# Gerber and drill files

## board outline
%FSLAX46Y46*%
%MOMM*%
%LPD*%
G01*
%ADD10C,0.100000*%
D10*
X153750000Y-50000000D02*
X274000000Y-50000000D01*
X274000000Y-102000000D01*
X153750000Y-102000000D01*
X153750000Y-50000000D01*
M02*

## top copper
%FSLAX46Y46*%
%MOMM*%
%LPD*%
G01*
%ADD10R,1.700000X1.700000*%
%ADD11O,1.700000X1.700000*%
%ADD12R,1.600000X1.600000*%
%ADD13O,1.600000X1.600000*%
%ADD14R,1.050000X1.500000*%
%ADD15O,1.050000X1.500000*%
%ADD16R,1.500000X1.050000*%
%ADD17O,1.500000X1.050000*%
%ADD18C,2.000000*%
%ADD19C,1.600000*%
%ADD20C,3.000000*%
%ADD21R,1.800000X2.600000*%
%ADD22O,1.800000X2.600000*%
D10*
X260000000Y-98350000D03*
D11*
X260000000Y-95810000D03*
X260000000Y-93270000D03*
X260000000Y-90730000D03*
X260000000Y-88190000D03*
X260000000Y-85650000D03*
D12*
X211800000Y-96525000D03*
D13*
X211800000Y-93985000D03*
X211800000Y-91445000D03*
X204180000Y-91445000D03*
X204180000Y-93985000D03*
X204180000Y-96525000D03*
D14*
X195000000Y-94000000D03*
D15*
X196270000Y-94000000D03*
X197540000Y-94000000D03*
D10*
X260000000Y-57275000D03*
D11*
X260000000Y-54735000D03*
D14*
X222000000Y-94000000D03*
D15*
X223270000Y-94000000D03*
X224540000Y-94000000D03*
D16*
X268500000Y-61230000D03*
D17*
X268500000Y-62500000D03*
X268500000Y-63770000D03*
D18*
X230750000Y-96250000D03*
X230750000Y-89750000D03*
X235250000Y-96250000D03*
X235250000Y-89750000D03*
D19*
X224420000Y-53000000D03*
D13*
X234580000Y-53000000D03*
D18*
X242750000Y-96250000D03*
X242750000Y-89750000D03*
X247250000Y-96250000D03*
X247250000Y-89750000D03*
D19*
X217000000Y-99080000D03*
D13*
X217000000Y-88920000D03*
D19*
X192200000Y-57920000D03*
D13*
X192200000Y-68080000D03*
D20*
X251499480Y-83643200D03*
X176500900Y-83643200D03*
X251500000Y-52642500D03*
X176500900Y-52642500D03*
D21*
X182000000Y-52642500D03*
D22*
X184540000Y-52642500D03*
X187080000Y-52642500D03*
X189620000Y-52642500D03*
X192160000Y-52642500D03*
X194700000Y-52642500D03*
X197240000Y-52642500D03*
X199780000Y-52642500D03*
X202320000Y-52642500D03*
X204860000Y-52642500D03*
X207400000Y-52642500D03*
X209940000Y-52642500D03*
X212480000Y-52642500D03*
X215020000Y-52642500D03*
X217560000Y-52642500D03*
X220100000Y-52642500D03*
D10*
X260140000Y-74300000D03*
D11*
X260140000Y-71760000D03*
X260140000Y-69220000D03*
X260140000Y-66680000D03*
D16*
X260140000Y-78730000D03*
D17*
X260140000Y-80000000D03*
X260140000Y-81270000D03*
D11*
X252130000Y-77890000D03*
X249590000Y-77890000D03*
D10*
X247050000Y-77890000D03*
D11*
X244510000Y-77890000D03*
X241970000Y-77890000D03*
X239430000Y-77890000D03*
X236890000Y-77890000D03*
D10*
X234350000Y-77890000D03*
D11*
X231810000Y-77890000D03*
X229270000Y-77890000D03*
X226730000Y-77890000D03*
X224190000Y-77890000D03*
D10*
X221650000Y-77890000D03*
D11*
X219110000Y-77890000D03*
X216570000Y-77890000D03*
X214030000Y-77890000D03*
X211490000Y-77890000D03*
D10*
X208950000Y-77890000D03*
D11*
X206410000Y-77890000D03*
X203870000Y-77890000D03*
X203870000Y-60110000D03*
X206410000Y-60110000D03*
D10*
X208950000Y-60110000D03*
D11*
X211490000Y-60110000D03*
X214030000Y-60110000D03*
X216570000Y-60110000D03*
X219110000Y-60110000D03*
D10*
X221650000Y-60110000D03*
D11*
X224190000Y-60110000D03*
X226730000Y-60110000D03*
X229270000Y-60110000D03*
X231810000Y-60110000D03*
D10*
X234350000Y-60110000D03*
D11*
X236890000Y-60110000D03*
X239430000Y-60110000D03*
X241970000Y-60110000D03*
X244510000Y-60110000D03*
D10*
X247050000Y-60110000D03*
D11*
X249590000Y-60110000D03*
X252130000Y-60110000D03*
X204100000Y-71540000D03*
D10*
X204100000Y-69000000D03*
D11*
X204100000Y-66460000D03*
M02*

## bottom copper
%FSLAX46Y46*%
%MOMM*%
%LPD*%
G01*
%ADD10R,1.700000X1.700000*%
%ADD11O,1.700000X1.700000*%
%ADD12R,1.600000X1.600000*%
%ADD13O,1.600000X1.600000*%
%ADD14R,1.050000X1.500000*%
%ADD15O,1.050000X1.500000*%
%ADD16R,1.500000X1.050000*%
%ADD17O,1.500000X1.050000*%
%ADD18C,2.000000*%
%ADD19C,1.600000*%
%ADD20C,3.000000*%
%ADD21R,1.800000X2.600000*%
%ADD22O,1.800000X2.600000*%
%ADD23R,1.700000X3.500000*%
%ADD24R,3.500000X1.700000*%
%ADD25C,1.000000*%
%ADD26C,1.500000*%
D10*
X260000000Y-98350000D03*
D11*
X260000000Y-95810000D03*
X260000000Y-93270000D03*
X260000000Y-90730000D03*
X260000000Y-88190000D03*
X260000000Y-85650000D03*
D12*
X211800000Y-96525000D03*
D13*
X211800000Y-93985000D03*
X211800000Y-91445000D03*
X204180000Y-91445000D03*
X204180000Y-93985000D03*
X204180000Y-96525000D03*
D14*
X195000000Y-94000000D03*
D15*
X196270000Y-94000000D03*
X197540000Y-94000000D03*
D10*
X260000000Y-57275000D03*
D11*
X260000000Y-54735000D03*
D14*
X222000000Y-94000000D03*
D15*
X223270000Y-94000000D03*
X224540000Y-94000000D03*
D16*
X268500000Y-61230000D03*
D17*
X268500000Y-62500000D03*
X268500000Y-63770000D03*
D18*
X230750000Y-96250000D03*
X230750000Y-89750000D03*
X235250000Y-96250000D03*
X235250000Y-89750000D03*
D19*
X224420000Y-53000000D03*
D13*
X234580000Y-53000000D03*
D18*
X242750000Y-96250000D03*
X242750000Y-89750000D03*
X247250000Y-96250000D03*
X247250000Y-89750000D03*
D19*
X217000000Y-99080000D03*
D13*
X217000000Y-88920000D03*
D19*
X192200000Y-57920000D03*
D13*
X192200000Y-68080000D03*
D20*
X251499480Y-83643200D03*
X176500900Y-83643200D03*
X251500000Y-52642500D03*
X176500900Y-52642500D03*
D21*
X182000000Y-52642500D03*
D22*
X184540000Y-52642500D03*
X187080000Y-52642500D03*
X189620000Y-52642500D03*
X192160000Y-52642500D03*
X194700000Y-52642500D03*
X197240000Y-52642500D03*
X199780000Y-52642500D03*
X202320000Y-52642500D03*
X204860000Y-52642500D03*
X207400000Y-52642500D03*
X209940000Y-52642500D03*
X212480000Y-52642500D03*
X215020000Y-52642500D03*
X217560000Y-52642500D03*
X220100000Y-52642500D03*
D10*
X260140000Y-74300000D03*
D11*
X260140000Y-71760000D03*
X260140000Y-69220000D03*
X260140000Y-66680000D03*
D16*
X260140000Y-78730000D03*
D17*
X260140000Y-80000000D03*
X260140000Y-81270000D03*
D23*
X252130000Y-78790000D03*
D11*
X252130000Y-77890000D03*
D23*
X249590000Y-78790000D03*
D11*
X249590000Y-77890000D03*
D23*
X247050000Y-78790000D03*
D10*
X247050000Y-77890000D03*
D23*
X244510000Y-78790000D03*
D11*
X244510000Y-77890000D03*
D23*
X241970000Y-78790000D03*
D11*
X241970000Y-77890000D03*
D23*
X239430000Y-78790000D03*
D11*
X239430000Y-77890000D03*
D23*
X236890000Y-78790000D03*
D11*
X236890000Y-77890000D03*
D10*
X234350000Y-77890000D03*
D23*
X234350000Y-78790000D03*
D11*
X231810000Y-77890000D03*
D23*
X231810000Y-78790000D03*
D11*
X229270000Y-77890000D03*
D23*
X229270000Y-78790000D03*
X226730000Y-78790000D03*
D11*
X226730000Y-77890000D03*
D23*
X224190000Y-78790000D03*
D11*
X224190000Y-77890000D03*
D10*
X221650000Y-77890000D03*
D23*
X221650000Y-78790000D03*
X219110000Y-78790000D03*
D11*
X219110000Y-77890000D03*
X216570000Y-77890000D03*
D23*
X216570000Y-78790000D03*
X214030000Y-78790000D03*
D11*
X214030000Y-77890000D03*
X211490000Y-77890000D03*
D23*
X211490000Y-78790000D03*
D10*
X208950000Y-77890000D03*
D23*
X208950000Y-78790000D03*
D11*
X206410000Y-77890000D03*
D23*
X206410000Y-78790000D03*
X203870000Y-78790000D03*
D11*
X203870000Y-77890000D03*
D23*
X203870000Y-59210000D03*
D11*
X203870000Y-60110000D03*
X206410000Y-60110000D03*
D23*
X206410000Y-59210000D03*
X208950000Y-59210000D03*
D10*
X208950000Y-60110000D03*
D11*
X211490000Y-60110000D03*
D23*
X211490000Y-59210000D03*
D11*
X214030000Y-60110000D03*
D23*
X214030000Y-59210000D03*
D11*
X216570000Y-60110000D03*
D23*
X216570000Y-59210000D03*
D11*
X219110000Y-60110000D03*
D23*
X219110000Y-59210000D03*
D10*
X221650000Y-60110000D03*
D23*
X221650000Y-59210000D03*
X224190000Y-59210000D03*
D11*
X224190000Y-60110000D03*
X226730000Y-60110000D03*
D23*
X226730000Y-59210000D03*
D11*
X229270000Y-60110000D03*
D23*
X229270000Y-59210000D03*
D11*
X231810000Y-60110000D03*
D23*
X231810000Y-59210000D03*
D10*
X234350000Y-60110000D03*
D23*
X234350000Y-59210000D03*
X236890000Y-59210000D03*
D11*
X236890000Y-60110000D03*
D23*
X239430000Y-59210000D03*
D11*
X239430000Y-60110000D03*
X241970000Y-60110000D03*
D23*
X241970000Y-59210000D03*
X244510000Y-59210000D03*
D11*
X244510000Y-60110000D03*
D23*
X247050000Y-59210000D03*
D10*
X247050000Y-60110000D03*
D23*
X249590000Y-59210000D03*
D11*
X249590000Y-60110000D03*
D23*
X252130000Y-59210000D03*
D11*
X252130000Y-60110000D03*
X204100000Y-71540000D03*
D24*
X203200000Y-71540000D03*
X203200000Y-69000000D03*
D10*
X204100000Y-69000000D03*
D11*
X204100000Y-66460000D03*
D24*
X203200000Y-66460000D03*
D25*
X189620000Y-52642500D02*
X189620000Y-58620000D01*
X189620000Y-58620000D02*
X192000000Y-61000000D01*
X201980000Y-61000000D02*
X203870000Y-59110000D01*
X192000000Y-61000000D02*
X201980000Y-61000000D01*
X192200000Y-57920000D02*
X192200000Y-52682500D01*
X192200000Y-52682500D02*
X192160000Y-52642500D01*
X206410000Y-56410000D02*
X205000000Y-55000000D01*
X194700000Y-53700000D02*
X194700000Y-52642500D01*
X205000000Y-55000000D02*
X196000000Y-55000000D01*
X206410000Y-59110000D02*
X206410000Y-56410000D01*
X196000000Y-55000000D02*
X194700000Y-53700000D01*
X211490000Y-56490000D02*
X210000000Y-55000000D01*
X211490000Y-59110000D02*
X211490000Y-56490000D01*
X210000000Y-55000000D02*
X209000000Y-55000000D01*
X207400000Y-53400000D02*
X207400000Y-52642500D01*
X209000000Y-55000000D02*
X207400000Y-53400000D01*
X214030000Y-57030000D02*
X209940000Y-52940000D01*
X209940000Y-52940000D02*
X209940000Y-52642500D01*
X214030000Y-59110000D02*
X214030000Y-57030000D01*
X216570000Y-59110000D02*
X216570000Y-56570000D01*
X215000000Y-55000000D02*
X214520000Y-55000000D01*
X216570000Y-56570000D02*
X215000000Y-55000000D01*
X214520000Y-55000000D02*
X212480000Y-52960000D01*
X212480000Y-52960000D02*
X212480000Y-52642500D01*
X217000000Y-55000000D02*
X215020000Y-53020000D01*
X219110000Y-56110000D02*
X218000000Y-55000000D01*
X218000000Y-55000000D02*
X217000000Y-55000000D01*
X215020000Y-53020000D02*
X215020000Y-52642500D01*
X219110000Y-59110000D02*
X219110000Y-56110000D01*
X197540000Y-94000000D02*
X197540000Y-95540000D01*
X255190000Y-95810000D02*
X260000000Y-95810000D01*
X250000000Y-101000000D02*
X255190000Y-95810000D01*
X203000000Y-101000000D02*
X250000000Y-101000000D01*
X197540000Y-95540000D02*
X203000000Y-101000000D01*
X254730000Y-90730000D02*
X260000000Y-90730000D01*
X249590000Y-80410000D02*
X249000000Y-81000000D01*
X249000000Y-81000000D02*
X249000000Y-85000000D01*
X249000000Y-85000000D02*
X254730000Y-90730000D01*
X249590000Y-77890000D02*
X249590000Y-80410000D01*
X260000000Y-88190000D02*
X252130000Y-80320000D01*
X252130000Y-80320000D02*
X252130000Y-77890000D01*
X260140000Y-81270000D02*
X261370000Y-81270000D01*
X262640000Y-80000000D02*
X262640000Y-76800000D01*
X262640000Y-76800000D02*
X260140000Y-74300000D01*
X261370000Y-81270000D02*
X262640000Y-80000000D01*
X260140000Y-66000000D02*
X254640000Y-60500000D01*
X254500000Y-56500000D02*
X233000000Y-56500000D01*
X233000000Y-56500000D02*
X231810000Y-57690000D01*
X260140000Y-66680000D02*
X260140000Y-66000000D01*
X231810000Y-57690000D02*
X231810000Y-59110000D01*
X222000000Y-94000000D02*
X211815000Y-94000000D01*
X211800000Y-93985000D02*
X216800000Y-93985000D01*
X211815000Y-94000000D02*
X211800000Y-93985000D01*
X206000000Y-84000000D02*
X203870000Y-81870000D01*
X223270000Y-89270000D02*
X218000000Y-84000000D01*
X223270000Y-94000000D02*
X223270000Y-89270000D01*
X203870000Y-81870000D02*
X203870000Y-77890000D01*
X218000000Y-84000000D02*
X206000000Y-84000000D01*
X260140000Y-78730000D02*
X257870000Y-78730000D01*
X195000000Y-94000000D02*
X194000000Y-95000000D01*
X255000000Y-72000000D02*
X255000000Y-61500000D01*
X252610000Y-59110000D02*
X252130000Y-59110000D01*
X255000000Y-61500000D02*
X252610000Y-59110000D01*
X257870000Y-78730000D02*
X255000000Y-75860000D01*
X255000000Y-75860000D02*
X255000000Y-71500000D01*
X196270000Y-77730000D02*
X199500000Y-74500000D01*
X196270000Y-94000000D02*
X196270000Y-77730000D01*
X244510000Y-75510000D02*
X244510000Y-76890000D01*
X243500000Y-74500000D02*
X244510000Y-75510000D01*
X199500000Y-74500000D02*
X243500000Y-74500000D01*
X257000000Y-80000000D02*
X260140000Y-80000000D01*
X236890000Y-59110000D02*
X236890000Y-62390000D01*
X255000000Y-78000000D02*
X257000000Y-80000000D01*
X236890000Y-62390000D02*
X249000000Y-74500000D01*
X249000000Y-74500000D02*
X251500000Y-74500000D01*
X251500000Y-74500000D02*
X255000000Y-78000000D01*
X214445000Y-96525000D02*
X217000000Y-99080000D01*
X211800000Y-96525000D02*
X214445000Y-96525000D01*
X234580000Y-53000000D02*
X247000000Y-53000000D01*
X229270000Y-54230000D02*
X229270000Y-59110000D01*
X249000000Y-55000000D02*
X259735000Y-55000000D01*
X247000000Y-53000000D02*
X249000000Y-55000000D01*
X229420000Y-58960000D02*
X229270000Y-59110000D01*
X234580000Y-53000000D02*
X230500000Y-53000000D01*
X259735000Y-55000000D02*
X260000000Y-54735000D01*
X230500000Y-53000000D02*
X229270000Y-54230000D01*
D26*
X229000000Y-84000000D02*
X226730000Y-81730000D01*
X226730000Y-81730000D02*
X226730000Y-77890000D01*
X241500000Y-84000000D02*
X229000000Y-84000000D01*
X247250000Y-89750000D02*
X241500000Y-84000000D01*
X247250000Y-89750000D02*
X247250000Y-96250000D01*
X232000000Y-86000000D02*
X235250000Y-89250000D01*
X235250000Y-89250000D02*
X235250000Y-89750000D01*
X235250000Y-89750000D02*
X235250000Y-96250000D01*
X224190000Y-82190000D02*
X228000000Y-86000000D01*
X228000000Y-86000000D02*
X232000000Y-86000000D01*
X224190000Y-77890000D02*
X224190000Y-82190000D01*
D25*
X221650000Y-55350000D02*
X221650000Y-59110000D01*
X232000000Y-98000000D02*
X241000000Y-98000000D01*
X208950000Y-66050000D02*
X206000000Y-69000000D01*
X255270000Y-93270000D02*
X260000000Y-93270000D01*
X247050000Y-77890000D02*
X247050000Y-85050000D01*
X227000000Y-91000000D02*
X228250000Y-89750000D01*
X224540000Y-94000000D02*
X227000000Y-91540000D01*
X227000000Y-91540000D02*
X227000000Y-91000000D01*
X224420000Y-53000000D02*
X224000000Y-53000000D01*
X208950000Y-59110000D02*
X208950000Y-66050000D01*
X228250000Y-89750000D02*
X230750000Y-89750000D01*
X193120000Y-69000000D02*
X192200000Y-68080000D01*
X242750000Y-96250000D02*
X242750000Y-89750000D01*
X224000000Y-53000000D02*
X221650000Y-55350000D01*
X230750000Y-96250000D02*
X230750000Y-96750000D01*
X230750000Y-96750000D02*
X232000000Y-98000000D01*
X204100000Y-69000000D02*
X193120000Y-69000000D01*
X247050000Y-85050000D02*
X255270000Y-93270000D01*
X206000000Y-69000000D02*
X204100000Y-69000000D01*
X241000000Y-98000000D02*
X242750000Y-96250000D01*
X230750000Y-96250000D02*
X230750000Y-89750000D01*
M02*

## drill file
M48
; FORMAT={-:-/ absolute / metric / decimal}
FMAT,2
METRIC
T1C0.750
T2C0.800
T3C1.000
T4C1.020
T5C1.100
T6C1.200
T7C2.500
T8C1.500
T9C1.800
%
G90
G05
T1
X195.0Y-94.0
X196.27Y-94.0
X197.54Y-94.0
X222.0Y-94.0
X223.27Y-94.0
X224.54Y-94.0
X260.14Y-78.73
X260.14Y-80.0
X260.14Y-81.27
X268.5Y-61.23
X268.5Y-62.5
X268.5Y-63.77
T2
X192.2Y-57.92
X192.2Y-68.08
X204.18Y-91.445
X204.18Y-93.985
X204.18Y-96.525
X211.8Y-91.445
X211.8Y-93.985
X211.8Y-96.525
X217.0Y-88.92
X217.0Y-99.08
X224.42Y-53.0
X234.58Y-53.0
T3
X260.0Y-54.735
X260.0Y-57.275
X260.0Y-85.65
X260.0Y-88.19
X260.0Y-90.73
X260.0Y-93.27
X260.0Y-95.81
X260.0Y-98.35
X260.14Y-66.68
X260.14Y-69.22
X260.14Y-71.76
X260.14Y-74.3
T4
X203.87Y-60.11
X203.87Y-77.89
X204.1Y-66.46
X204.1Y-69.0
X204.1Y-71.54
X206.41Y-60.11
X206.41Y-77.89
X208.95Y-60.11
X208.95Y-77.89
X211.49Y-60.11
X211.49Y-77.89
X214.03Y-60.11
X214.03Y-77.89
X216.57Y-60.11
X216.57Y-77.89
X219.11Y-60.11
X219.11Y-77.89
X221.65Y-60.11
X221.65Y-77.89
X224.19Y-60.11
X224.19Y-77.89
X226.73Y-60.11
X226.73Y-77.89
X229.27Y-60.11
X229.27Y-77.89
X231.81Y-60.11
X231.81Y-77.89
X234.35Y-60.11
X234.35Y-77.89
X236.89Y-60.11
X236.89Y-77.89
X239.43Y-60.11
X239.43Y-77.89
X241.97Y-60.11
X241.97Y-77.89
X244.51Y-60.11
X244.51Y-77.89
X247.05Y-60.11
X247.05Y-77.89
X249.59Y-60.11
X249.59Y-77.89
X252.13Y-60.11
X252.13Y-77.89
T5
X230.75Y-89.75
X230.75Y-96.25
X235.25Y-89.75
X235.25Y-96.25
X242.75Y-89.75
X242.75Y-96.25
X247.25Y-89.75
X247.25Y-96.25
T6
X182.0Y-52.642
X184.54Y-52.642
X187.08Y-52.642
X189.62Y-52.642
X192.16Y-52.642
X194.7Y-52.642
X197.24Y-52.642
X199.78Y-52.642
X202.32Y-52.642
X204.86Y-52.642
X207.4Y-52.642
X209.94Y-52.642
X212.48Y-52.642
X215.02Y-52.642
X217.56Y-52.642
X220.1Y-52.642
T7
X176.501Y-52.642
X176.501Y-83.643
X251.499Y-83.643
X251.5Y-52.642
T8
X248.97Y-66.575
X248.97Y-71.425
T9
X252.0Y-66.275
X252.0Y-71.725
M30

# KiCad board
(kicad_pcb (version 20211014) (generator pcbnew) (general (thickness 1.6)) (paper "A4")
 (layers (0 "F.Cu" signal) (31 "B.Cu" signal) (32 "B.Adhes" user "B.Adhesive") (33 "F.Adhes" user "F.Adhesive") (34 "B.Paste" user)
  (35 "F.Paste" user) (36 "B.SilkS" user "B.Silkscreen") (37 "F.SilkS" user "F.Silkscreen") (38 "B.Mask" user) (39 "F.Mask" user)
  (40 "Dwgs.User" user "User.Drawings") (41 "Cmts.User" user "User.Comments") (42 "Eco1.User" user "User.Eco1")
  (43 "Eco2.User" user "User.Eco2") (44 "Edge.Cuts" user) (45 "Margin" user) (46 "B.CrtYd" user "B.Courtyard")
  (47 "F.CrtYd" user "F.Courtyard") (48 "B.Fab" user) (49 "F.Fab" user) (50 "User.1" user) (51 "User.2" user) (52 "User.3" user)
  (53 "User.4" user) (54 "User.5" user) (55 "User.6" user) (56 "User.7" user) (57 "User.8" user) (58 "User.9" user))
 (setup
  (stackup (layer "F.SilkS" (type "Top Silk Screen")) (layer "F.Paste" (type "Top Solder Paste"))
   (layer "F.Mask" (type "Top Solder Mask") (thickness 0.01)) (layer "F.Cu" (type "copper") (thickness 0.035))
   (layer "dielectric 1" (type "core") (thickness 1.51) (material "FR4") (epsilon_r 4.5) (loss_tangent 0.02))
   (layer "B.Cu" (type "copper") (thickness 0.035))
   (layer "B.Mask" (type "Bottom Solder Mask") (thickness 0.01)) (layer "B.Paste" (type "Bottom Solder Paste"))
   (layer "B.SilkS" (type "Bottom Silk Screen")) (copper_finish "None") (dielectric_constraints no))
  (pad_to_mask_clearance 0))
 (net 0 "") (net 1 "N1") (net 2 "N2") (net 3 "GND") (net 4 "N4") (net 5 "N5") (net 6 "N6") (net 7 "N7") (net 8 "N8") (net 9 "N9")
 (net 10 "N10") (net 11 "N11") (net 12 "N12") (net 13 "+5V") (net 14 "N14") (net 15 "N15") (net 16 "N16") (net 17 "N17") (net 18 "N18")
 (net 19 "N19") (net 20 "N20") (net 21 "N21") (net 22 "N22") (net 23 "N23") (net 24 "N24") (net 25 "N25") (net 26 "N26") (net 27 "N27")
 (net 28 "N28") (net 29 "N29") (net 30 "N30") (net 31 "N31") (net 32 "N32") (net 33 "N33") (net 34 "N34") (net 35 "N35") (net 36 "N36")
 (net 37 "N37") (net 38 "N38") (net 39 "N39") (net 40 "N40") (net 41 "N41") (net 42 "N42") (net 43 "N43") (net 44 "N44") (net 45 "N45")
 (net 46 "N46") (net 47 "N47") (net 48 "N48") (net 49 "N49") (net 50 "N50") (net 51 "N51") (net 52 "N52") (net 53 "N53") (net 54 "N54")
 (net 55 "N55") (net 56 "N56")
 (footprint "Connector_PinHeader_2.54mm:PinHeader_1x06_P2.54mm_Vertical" (layer "F.Cu") (at 260 98.35 180)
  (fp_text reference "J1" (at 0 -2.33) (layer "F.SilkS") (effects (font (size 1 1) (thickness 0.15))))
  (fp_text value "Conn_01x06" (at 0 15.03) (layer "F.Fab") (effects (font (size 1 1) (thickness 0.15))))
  (pad "1" thru_hole rect (at 0 0 180) (size 1.7 1.7) (drill 1) (layers *.Cu *.Mask) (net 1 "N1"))
  (pad "2" thru_hole oval (at 0 2.54 180) (size 1.7 1.7) (drill 1) (layers *.Cu *.Mask) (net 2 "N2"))
  (pad "3" thru_hole oval (at 0 5.08 180) (size 1.7 1.7) (drill 1) (layers *.Cu *.Mask) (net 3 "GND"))
  (pad "4" thru_hole oval (at 0 7.62 180) (size 1.7 1.7) (drill 1) (layers *.Cu *.Mask) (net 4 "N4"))
  (pad "5" thru_hole oval (at 0 10.16 180) (size 1.7 1.7) (drill 1) (layers *.Cu *.Mask) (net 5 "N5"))
  (pad "6" thru_hole oval (at 0 12.7 180) (size 1.7 1.7) (drill 1) (layers *.Cu *.Mask) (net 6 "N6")))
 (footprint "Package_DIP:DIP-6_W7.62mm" (layer "F.Cu") (at 211.8 96.525 180)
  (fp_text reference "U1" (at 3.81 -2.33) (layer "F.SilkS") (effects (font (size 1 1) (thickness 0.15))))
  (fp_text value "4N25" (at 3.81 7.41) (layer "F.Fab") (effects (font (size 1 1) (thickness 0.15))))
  (pad "1" thru_hole rect (at 0 0 180) (size 1.6 1.6) (drill 0.8) (layers *.Cu *.Mask) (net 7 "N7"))
  (pad "2" thru_hole oval (at 0 2.54 180) (size 1.6 1.6) (drill 0.8) (layers *.Cu *.Mask) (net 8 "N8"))
  (pad "3" thru_hole oval (at 0 5.08 180) (size 1.6 1.6) (drill 0.8) (layers *.Cu *.Mask) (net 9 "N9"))
  (pad "4" thru_hole oval (at 7.62 5.08 180) (size 1.6 1.6) (drill 0.8) (layers *.Cu *.Mask) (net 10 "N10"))
  (pad "5" thru_hole oval (at 7.62 2.54 180) (size 1.6 1.6) (drill 0.8) (layers *.Cu *.Mask) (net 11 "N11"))
  (pad "6" thru_hole oval (at 7.62 0 180) (size 1.6 1.6) (drill 0.8) (layers *.Cu *.Mask) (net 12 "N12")))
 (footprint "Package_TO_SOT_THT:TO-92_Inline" (layer "F.Cu") (at 195 94)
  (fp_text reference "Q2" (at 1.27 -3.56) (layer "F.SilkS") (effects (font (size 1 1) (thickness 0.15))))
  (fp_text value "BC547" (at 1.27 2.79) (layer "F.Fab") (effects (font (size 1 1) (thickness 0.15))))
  (pad "1" thru_hole rect (at 0 0) (size 1.05 1.5) (drill 0.75) (layers *.Cu *.Mask) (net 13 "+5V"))
  (pad "2" thru_hole oval (at 1.27 0) (size 1.05 1.5) (drill 0.75) (layers *.Cu *.Mask) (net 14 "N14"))
  (pad "3" thru_hole oval (at 2.54 0) (size 1.05 1.5) (drill 0.75) (layers *.Cu *.Mask) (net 2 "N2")))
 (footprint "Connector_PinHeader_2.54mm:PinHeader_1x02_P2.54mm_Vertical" (layer "F.Cu") (at 260 57.275 180)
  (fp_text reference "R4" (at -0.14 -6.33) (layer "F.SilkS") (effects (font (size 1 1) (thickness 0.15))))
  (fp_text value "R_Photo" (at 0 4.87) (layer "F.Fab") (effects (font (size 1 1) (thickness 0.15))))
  (pad "1" thru_hole rect (at 0 0 180) (size 1.7 1.7) (drill 1) (layers *.Cu *.Mask) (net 13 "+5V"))
  (pad "2" thru_hole oval (at 0 2.54 180) (size 1.7 1.7) (drill 1) (layers *.Cu *.Mask) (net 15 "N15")))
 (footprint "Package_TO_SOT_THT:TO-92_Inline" (layer "F.Cu") (at 222 94)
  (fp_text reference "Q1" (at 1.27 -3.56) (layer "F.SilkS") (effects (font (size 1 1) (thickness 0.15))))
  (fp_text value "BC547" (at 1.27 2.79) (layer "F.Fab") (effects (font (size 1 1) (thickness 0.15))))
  (pad "1" thru_hole rect (at 0 0) (size 1.05 1.5) (drill 0.75) (layers *.Cu *.Mask) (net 8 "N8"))
  (pad "2" thru_hole oval (at 1.27 0) (size 1.05 1.5) (drill 0.75) (layers *.Cu *.Mask) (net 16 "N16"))
  (pad "3" thru_hole oval (at 2.54 0) (size 1.05 1.5) (drill 0.75) (layers *.Cu *.Mask) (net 3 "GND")))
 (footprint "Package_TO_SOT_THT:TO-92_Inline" (layer "F.Cu") (at 268.5 61.23 -90)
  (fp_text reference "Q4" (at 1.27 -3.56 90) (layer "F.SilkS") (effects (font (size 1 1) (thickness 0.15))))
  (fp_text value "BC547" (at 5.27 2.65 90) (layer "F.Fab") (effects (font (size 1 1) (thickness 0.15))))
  (pad "1" thru_hole rect (at 0 0 270) (size 1.05 1.5) (drill 0.75) (layers *.Cu *.Mask) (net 13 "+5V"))
  (pad "2" thru_hole oval (at 1.27 0 270) (size 1.05 1.5) (drill 0.75) (layers *.Cu *.Mask) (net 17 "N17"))
  (pad "3" thru_hole oval (at 2.54 0 270) (size 1.05 1.5) (drill 0.75) (layers *.Cu *.Mask) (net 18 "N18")))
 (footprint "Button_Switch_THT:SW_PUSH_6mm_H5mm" (layer "F.Cu") (at 230.75 96.25 90)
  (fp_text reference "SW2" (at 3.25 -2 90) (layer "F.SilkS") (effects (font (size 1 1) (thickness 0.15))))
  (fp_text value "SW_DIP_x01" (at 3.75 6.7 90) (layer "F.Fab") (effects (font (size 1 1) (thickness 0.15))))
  (pad "1" thru_hole circle (at 0 0 180) (size 2 2) (drill 1.1) (layers *.Cu *.Mask) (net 3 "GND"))
  (pad "1" thru_hole circle (at 6.5 0 180) (size 2 2) (drill 1.1) (layers *.Cu *.Mask) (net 3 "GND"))
  (pad "2" thru_hole circle (at 0 4.5 180) (size 2 2) (drill 1.1) (layers *.Cu *.Mask) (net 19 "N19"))
  (pad "2" thru_hole circle (at 6.5 4.5 180) (size 2 2) (drill 1.1) (layers *.Cu *.Mask) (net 19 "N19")))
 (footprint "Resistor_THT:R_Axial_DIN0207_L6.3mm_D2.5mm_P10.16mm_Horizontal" (layer "F.Cu") (at 224.42 53)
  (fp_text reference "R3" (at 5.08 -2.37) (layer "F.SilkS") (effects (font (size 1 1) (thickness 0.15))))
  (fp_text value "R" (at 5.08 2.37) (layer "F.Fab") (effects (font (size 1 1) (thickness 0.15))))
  (pad "1" thru_hole circle (at 0 0) (size 1.6 1.6) (drill 0.8) (layers *.Cu *.Mask) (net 3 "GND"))
  (pad "2" thru_hole oval (at 10.16 0) (size 1.6 1.6) (drill 0.8) (layers *.Cu *.Mask) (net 15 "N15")))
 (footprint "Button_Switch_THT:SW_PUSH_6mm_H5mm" (layer "F.Cu") (at 242.75 96.25 90)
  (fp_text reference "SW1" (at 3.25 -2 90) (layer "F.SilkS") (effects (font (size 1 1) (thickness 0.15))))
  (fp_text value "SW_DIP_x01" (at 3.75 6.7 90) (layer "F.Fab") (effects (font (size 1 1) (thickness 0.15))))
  (pad "1" thru_hole circle (at 0 0 180) (size 2 2) (drill 1.1) (layers *.Cu *.Mask) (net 3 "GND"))
  (pad "1" thru_hole circle (at 6.5 0 180) (size 2 2) (drill 1.1) (layers *.Cu *.Mask) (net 3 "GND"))
  (pad "2" thru_hole circle (at 0 4.5 180) (size 2 2) (drill 1.1) (layers *.Cu *.Mask) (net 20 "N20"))
  (pad "2" thru_hole circle (at 6.5 4.5 180) (size 2 2) (drill 1.1) (layers *.Cu *.Mask) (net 20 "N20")))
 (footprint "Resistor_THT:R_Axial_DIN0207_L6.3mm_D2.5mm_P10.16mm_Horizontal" (layer "F.Cu") (at 217 99.08 90)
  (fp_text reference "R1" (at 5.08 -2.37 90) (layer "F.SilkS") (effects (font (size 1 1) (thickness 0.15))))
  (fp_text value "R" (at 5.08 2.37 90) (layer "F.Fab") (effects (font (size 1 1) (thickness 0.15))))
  (pad "1" thru_hole circle (at 0 0 90) (size 1.6 1.6) (drill 0.8) (layers *.Cu *.Mask) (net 7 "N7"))
  (pad "2" thru_hole oval (at 10.16 0 90) (size 1.6 1.6) (drill 0.8) (layers *.Cu *.Mask) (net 13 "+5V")))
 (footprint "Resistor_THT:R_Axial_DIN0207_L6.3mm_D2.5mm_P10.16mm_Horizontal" (layer "F.Cu") (at 192.2 57.92 -90)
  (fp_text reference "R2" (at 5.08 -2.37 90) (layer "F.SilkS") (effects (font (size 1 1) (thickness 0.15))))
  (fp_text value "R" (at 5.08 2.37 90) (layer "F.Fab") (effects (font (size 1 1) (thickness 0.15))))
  (pad "1" thru_hole circle (at 0 0 270) (size 1.6 1.6) (drill 0.8) (layers *.Cu *.Mask) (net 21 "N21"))
  (pad "2" thru_hole oval (at 10.16 0 270) (size 1.6 1.6) (drill 0.8) (layers *.Cu *.Mask) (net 3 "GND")))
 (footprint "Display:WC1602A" (layer "F.Cu") (at 182 52.6425)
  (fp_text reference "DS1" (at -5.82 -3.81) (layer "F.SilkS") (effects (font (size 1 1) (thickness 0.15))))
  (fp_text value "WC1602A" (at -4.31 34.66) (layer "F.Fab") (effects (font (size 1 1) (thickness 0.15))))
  (pad "" thru_hole circle (at 69.49948 31.0007) (size 3 3) (drill 2.5) (layers *.Cu *.Mask))
  (pad "" thru_hole circle (at -5.4991 31.0007) (size 3 3) (drill 2.5) (layers *.Cu *.Mask))
  (pad "" thru_hole circle (at 69.5 0) (size 3 3) (drill 2.5) (layers *.Cu *.Mask))
  (pad "" thru_hole circle (at -5.4991 0) (size 3 3) (drill 2.5) (layers *.Cu *.Mask))
  (pad "1" thru_hole rect (at 0 0) (size 1.8 2.6) (drill 1.2) (layers *.Cu *.Mask) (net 3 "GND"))
  (pad "2" thru_hole oval (at 2.54 0) (size 1.8 2.6) (drill 1.2) (layers *.Cu *.Mask) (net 18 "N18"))
  (pad "3" thru_hole oval (at 5.08 0) (size 1.8 2.6) (drill 1.2) (layers *.Cu *.Mask) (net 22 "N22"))
  (pad "4" thru_hole oval (at 7.62 0) (size 1.8 2.6) (drill 1.2) (layers *.Cu *.Mask) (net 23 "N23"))
  (pad "5" thru_hole oval (at 10.16 0) (size 1.8 2.6) (drill 1.2) (layers *.Cu *.Mask) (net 21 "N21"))
  (pad "6" thru_hole oval (at 12.7 0) (size 1.8 2.6) (drill 1.2) (layers *.Cu *.Mask) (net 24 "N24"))
  (pad "7" thru_hole oval (at 15.24 0) (size 1.8 2.6) (drill 1.2) (layers *.Cu *.Mask) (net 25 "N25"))
  (pad "8" thru_hole oval (at 17.78 0) (size 1.8 2.6) (drill 1.2) (layers *.Cu *.Mask) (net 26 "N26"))
  (pad "9" thru_hole oval (at 20.32 0) (size 1.8 2.6) (drill 1.2) (layers *.Cu *.Mask) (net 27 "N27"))
  (pad "10" thru_hole oval (at 22.86 0) (size 1.8 2.6) (drill 1.2) (layers *.Cu *.Mask) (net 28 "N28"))
  (pad "11" thru_hole oval (at 25.4 0) (size 1.8 2.6) (drill 1.2) (layers *.Cu *.Mask) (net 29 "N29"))
  (pad "12" thru_hole oval (at 27.94 0) (size 1.8 2.6) (drill 1.2) (layers *.Cu *.Mask) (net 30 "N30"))
  (pad "13" thru_hole oval (at 30.48 0) (size 1.8 2.6) (drill 1.2) (layers *.Cu *.Mask) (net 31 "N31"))
  (pad "14" thru_hole oval (at 33.02 0) (size 1.8 2.6) (drill 1.2) (layers *.Cu *.Mask) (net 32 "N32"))
  (pad "15" thru_hole oval (at 35.56 0) (size 1.8 2.6) (drill 1.2) (layers *.Cu *.Mask) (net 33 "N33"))
  (pad "16" thru_hole oval (at 38.1 0) (size 1.8 2.6) (drill 1.2) (layers *.Cu *.Mask) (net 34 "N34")))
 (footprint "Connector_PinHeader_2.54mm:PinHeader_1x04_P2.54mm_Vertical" (layer "F.Cu") (at 260.14 74.3 180)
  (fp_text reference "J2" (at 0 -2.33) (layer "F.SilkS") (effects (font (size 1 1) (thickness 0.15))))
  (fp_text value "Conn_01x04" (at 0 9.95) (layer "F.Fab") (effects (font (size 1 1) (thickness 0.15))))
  (pad "1" thru_hole rect (at 0 0 180) (size 1.7 1.7) (drill 1) (layers *.Cu *.Mask) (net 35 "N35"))
  (pad "2" thru_hole oval (at 0 2.54 180) (size 1.7 1.7) (drill 1) (layers *.Cu *.Mask) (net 3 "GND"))
  (pad "3" thru_hole oval (at 0 5.08 180) (size 1.7 1.7) (drill 1) (layers *.Cu *.Mask) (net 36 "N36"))
  (pad "4" thru_hole oval (at 0 7.62 180) (size 1.7 1.7) (drill 1) (layers *.Cu *.Mask) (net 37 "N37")))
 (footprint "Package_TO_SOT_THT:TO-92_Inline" (layer "F.Cu") (at 260.14 78.73 -90)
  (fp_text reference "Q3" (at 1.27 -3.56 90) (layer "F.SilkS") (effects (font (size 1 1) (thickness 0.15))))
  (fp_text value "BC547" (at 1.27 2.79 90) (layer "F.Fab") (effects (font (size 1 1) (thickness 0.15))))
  (pad "1" thru_hole rect (at 0 0 270) (size 1.05 1.5) (drill 0.75) (layers *.Cu *.Mask) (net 13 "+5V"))
  (pad "2" thru_hole oval (at 1.27 0 270) (size 1.05 1.5) (drill 0.75) (layers *.Cu *.Mask) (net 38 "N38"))
  (pad "3" thru_hole oval (at 2.54 0 270) (size 1.05 1.5) (drill 0.75) (layers *.Cu *.Mask) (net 35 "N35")))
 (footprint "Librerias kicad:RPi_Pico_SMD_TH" (layer "B.Cu") (at 228 69 90)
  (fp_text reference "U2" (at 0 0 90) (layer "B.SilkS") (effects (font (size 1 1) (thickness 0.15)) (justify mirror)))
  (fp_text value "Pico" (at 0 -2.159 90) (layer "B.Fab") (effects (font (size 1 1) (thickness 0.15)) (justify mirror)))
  (pad "" np_thru_hole oval (at -2.725 24 90) (size 1.8 1.8) (drill 1.8) (layers *.Cu *.Mask))
  (pad "" np_thru_hole oval (at -2.425 20.97 90) (size 1.5 1.5) (drill 1.5) (layers *.Cu *.Mask))
  (pad "" np_thru_hole oval (at 2.425 20.97 90) (size 1.5 1.5) (drill 1.5) (layers *.Cu *.Mask))
  (pad "" np_thru_hole oval (at 2.725 24 90) (size 1.8 1.8) (drill 1.8) (layers *.Cu *.Mask))
  (pad "1" smd rect (at -8.89 24.13 90) (size 3.5 1.7) (drill (offset -0.9 0)) (layers "B.Cu" "B.Mask") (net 5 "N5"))
  (pad "1" thru_hole oval (at -8.89 24.13 90) (size 1.7 1.7) (drill 1.02) (layers *.Cu *.Mask) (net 5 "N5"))
  (pad "2" smd rect (at -8.89 21.59 90) (size 3.5 1.7) (drill (offset -0.9 0)) (layers "B.Cu" "B.Mask") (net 4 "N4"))
  (pad "2" thru_hole oval (at -8.89 21.59 90) (size 1.7 1.7) (drill 1.02) (layers *.Cu *.Mask) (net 4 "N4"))
  (pad "3" smd rect (at -8.89 19.05 90) (size 3.5 1.7) (drill (offset -0.9 0)) (layers "B.Cu" "B.Mask") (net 3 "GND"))
  (pad "3" thru_hole rect (at -8.89 19.05 90) (size 1.7 1.7) (drill 1.02) (layers *.Cu *.Mask) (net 3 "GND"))
  (pad "4" smd rect (at -8.89 16.51 90) (size 3.5 1.7) (drill (offset -0.9 0)) (layers "B.Cu" "B.Mask") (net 14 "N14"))
  (pad "4" thru_hole oval (at -8.89 16.51 90) (size 1.7 1.7) (drill 1.02) (layers *.Cu *.Mask) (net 14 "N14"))
  (pad "5" smd rect (at -8.89 13.97 90) (size 3.5 1.7) (drill (offset -0.9 0)) (layers "B.Cu" "B.Mask") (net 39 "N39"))
  (pad "5" thru_hole oval (at -8.89 13.97 90) (size 1.7 1.7) (drill 1.02) (layers *.Cu *.Mask) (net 39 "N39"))
  (pad "6" smd rect (at -8.89 11.43 90) (size 3.5 1.7) (drill (offset -0.9 0)) (layers "B.Cu" "B.Mask") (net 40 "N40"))
  (pad "6" thru_hole oval (at -8.89 11.43 90) (size 1.7 1.7) (drill 1.02) (layers *.Cu *.Mask) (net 40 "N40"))
  (pad "7" smd rect (at -8.89 8.89 90) (size 3.5 1.7) (drill (offset -0.9 0)) (layers "B.Cu" "B.Mask") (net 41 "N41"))
  (pad "7" thru_hole oval (at -8.89 8.89 90) (size 1.7 1.7) (drill 1.02) (layers *.Cu *.Mask) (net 41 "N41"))
  (pad "8" thru_hole rect (at -8.89 6.35 90) (size 1.7 1.7) (drill 1.02) (layers *.Cu *.Mask) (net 3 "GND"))
  (pad "8" smd rect (at -8.89 6.35 90) (size 3.5 1.7) (drill (offset -0.9 0)) (layers "B.Cu" "B.Mask") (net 3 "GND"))
  (pad "9" thru_hole oval (at -8.89 3.81 90) (size 1.7 1.7) (drill 1.02) (layers *.Cu *.Mask) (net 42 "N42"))
  (pad "9" smd rect (at -8.89 3.81 90) (size 3.5 1.7) (drill (offset -0.9 0)) (layers "B.Cu" "B.Mask") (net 42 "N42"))
  (pad "10" thru_hole oval (at -8.89 1.27 90) (size 1.7 1.7) (drill 1.02) (layers *.Cu *.Mask) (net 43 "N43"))
  (pad "10" smd rect (at -8.89 1.27 90) (size 3.5 1.7) (drill (offset -0.9 0)) (layers "B.Cu" "B.Mask") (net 43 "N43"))
  (pad "11" smd rect (at -8.89 -1.27 90) (size 3.5 1.7) (drill (offset -0.9 0)) (layers "B.Cu" "B.Mask") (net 20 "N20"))
  (pad "11" thru_hole oval (at -8.89 -1.27 90) (size 1.7 1.7) (drill 1.02) (layers *.Cu *.Mask) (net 20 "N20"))
  (pad "12" smd rect (at -8.89 -3.81 90) (size 3.5 1.7) (drill (offset -0.9 0)) (layers "B.Cu" "B.Mask") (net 19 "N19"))
  (pad "12" thru_hole oval (at -8.89 -3.81 90) (size 1.7 1.7) (drill 1.02) (layers *.Cu *.Mask) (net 19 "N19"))
  (pad "13" thru_hole rect (at -8.89 -6.35 90) (size 1.7 1.7) (drill 1.02) (layers *.Cu *.Mask) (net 3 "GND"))
  (pad "13" smd rect (at -8.89 -6.35 90) (size 3.5 1.7) (drill (offset -0.9 0)) (layers "B.Cu" "B.Mask") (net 3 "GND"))
  (pad "14" smd rect (at -8.89 -8.89 90) (size 3.5 1.7) (drill (offset -0.9 0)) (layers "B.Cu" "B.Mask") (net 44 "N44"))
  (pad "14" thru_hole oval (at -8.89 -8.89 90) (size 1.7 1.7) (drill 1.02) (layers *.Cu *.Mask) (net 44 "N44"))
  (pad "15" thru_hole oval (at -8.89 -11.43 90) (size 1.7 1.7) (drill 1.02) (layers *.Cu *.Mask) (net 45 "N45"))
  (pad "15" smd rect (at -8.89 -11.43 90) (size 3.5 1.7) (drill (offset -0.9 0)) (layers "B.Cu" "B.Mask") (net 45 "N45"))
  (pad "16" smd rect (at -8.89 -13.97 90) (size 3.5 1.7) (drill (offset -0.9 0)) (layers "B.Cu" "B.Mask") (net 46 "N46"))
  (pad "16" thru_hole oval (at -8.89 -13.97 90) (size 1.7 1.7) (drill 1.02) (layers *.Cu *.Mask) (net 46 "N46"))
  (pad "17" thru_hole oval (at -8.89 -16.51 90) (size 1.7 1.7) (drill 1.02) (layers *.Cu *.Mask) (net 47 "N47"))
  (pad "17" smd rect (at -8.89 -16.51 90) (size 3.5 1.7) (drill (offset -0.9 0)) (layers "B.Cu" "B.Mask") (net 47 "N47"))
  (pad "18" thru_hole rect (at -8.89 -19.05 90) (size 1.7 1.7) (drill 1.02) (layers *.Cu *.Mask) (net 3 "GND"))
  (pad "18" smd rect (at -8.89 -19.05 90) (size 3.5 1.7) (drill (offset -0.9 0)) (layers "B.Cu" "B.Mask") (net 3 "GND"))
  (pad "19" thru_hole oval (at -8.89 -21.59 90) (size 1.7 1.7) (drill 1.02) (layers *.Cu *.Mask) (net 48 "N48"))
  (pad "19" smd rect (at -8.89 -21.59 90) (size 3.5 1.7) (drill (offset -0.9 0)) (layers "B.Cu" "B.Mask") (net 48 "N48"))
  (pad "20" smd rect (at -8.89 -24.13 90) (size 3.5 1.7) (drill (offset -0.9 0)) (layers "B.Cu" "B.Mask") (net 16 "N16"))
  (pad "20" thru_hole oval (at -8.89 -24.13 90) (size 1.7 1.7) (drill 1.02) (layers *.Cu *.Mask) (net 16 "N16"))
  (pad "21" smd rect (at 8.89 -24.13 90) (size 3.5 1.7) (drill (offset 0.9 0)) (layers "B.Cu" "B.Mask") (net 23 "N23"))
  (pad "21" thru_hole oval (at 8.89 -24.13 90) (size 1.7 1.7) (drill 1.02) (layers *.Cu *.Mask) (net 23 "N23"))
  (pad "22" thru_hole oval (at 8.89 -21.59 90) (size 1.7 1.7) (drill 1.02) (layers *.Cu *.Mask) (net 24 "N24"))
  (pad "22" smd rect (at 8.89 -21.59 90) (size 3.5 1.7) (drill (offset 0.9 0)) (layers "B.Cu" "B.Mask") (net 24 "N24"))
  (pad "23" smd rect (at 8.89 -19.05 90) (size 3.5 1.7) (drill (offset 0.9 0)) (layers "B.Cu" "B.Mask") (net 3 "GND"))
  (pad "23" thru_hole rect (at 8.89 -19.05 90) (size 1.7 1.7) (drill 1.02) (layers *.Cu *.Mask) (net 3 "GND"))
  (pad "24" thru_hole oval (at 8.89 -16.51 90) (size 1.7 1.7) (drill 1.02) (layers *.Cu *.Mask) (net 29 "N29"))
  (pad "24" smd rect (at 8.89 -16.51 90) (size 3.5 1.7) (drill (offset 0.9 0)) (layers "B.Cu" "B.Mask") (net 29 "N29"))
  (pad "25" thru_hole oval (at 8.89 -13.97 90) (size 1.7 1.7) (drill 1.02) (layers *.Cu *.Mask) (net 30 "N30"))
  (pad "25" smd rect (at 8.89 -13.97 90) (size 3.5 1.7) (drill (offset 0.9 0)) (layers "B.Cu" "B.Mask") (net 30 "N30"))
  (pad "26" thru_hole oval (at 8.89 -11.43 90) (size 1.7 1.7) (drill 1.02) (layers *.Cu *.Mask) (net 31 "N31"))
  (pad "26" smd rect (at 8.89 -11.43 90) (size 3.5 1.7) (drill (offset 0.9 0)) (layers "B.Cu" "B.Mask") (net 31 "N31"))
  (pad "27" thru_hole oval (at 8.89 -8.89 90) (size 1.7 1.7) (drill 1.02) (layers *.Cu *.Mask) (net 32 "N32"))
  (pad "27" smd rect (at 8.89 -8.89 90) (size 3.5 1.7) (drill (offset 0.9 0)) (layers "B.Cu" "B.Mask") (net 32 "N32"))
  (pad "28" thru_hole rect (at 8.89 -6.35 90) (size 1.7 1.7) (drill 1.02) (layers *.Cu *.Mask) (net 3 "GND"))
  (pad "28" smd rect (at 8.89 -6.35 90) (size 3.5 1.7) (drill (offset 0.9 0)) (layers "B.Cu" "B.Mask") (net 3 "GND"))
  (pad "29" smd rect (at 8.89 -3.81 90) (size 3.5 1.7) (drill (offset 0.9 0)) (layers "B.Cu" "B.Mask") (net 17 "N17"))
  (pad "29" thru_hole oval (at 8.89 -3.81 90) (size 1.7 1.7) (drill 1.02) (layers *.Cu *.Mask) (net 17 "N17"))
  (pad "30" thru_hole oval (at 8.89 -1.27 90) (size 1.7 1.7) (drill 1.02) (layers *.Cu *.Mask) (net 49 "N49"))
  (pad "30" smd rect (at 8.89 -1.27 90) (size 3.5 1.7) (drill (offset 0.9 0)) (layers "B.Cu" "B.Mask") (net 49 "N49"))
  (pad "31" thru_hole oval (at 8.89 1.27 90) (size 1.7 1.7) (drill 1.02) (layers *.Cu *.Mask) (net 15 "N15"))
  (pad "31" smd rect (at 8.89 1.27 90) (size 3.5 1.7) (drill (offset 0.9 0)) (layers "B.Cu" "B.Mask") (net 15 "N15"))
  (pad "32" thru_hole oval (at 8.89 3.81 90) (size 1.7 1.7) (drill 1.02) (layers *.Cu *.Mask) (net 37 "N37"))
  (pad "32" smd rect (at 8.89 3.81 90) (size 3.5 1.7) (drill (offset 0.9 0)) (layers "B.Cu" "B.Mask") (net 37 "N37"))
  (pad "33" thru_hole rect (at 8.89 6.35 90) (size 1.7 1.7) (drill 1.02) (layers *.Cu *.Mask) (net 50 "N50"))
  (pad "33" smd rect (at 8.89 6.35 90) (size 3.5 1.7) (drill (offset 0.9 0)) (layers "B.Cu" "B.Mask") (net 50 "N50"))
  (pad "34" smd rect (at 8.89 8.89 90) (size 3.5 1.7) (drill (offset 0.9 0)) (layers "B.Cu" "B.Mask") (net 38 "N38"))
  (pad "34" thru_hole oval (at 8.89 8.89 90) (size 1.7 1.7) (drill 1.02) (layers *.Cu *.Mask) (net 38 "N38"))
  (pad "35" smd rect (at 8.89 11.43 90) (size 3.5 1.7) (drill (offset 0.9 0)) (layers "B.Cu" "B.Mask") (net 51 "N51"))
  (pad "35" thru_hole oval (at 8.89 11.43 90) (size 1.7 1.7) (drill 1.02) (layers *.Cu *.Mask) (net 51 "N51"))
  (pad "36" thru_hole oval (at 8.89 13.97 90) (size 1.7 1.7) (drill 1.02) (layers *.Cu *.Mask) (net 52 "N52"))
  (pad "36" smd rect (at 8.89 13.97 90) (size 3.5 1.7) (drill (offset 0.9 0)) (layers "B.Cu" "B.Mask") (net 52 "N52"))
  (pad "37" smd rect (at 8.89 16.51 90) (size 3.5 1.7) (drill (offset 0.9 0)) (layers "B.Cu" "B.Mask") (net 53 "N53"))
  (pad "37" thru_hole oval (at 8.89 16.51 90) (size 1.7 1.7) (drill 1.02) (layers *.Cu *.Mask) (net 53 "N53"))
  (pad "38" smd rect (at 8.89 19.05 90) (size 3.5 1.7) (drill (offset 0.9 0)) (layers "B.Cu" "B.Mask") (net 3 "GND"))
  (pad "38" thru_hole rect (at 8.89 19.05 90) (size 1.7 1.7) (drill 1.02) (layers *.Cu *.Mask) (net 3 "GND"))
  (pad "39" smd rect (at 8.89 21.59 90) (size 3.5 1.7) (drill (offset 0.9 0)) (layers "B.Cu" "B.Mask") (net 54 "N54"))
  (pad "39" thru_hole oval (at 8.89 21.59 90) (size 1.7 1.7) (drill 1.02) (layers *.Cu *.Mask) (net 54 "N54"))
  (pad "40" smd rect (at 8.89 24.13 90) (size 3.5 1.7) (drill (offset 0.9 0)) (layers "B.Cu" "B.Mask") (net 13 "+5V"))
  (pad "40" thru_hole oval (at 8.89 24.13 90) (size 1.7 1.7) (drill 1.02) (layers *.Cu *.Mask) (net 13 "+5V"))
  (pad "41" thru_hole oval (at -2.54 -23.9 90) (size 1.7 1.7) (drill 1.02) (layers *.Cu *.Mask) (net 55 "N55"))
  (pad "41" smd rect (at -2.54 -23.9) (size 3.5 1.7) (drill (offset -0.9 0)) (layers "B.Cu" "B.Mask") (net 55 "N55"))
  (pad "42" smd rect (at 0 -23.9) (size 3.5 1.7) (drill (offset -0.9 0)) (layers "B.Cu" "B.Mask") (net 3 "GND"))
  (pad "42" thru_hole rect (at 0 -23.9 90) (size 1.7 1.7) (drill 1.02) (layers *.Cu *.Mask) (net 3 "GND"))
  (pad "43" thru_hole oval (at 2.54 -23.9 90) (size 1.7 1.7) (drill 1.02) (layers *.Cu *.Mask) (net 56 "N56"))
  (pad "43" smd rect (at 2.54 -23.9) (size 3.5 1.7) (drill (offset -0.9 0)) (layers "B.Cu" "B.Mask") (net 56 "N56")))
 (gr_rect (start 153.75 50) (end 274 102) (layer "Edge.Cuts") (width 0.1) (fill none))
 (segment (start 189.62 52.6425) (end 189.62 58.62) (width 1) (layer "B.Cu") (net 23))
 (segment (start 189.62 58.62) (end 192 61) (width 1) (layer "B.Cu") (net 23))
 (segment (start 201.98 61) (end 203.87 59.11) (width 1) (layer "B.Cu") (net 23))
 (segment (start 192 61) (end 201.98 61) (width 1) (layer "B.Cu") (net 23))
 (segment (start 192.2 57.92) (end 192.2 52.6825) (width 1) (layer "B.Cu") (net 21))
 (segment (start 192.2 52.6825) (end 192.16 52.6425) (width 1) (layer "B.Cu") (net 21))
 (segment (start 206.41 56.41) (end 205 55) (width 1) (layer "B.Cu") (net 24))
 (segment (start 194.7 53.7) (end 194.7 52.6425) (width 1) (layer "B.Cu") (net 24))
 (segment (start 205 55) (end 196 55) (width 1) (layer "B.Cu") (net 24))
 (segment (start 206.41 59.11) (end 206.41 56.41) (width 1) (layer "B.Cu") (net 24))
 (segment (start 196 55) (end 194.7 53.7) (width 1) (layer "B.Cu") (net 24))
 (segment (start 211.49 56.49) (end 210 55) (width 1) (layer "B.Cu") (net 29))
 (segment (start 211.49 59.11) (end 211.49 56.49) (width 1) (layer "B.Cu") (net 29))
 (segment (start 210 55) (end 209 55) (width 1) (layer "B.Cu") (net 29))
 (segment (start 207.4 53.4) (end 207.4 52.6425) (width 1) (layer "B.Cu") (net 29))
 (segment (start 209 55) (end 207.4 53.4) (width 1) (layer "B.Cu") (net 29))
 (segment (start 214.03 57.03) (end 209.94 52.94) (width 1) (layer "B.Cu") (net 30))
 (segment (start 209.94 52.94) (end 209.94 52.6425) (width 1) (layer "B.Cu") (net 30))
 (segment (start 214.03 59.11) (end 214.03 57.03) (width 1) (layer "B.Cu") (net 30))
 (segment (start 216.57 59.11) (end 216.57 56.57) (width 1) (layer "B.Cu") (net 31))
 (segment (start 215 55) (end 214.52 55) (width 1) (layer "B.Cu") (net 31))
 (segment (start 216.57 56.57) (end 215 55) (width 1) (layer "B.Cu") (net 31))
 (segment (start 214.52 55) (end 212.48 52.96) (width 1) (layer "B.Cu") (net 31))
 (segment (start 212.48 52.96) (end 212.48 52.6425) (width 1) (layer "B.Cu") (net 31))
 (segment (start 217 55) (end 215.02 53.02) (width 1) (layer "B.Cu") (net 32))
 (segment (start 219.11 56.11) (end 218 55) (width 1) (layer "B.Cu") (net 32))
 (segment (start 218 55) (end 217 55) (width 1) (layer "B.Cu") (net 32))
 (segment (start 215.02 53.02) (end 215.02 52.6425) (width 1) (layer "B.Cu") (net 32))
 (segment (start 219.11 59.11) (end 219.11 56.11) (width 1) (layer "B.Cu") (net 32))
 (segment (start 197.54 94) (end 197.54 95.54) (width 1) (layer "B.Cu") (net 2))
 (segment (start 255.19 95.81) (end 260 95.81) (width 1) (layer "B.Cu") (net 2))
 (segment (start 250 101) (end 255.19 95.81) (width 1) (layer "B.Cu") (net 2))
 (segment (start 203 101) (end 250 101) (width 1) (layer "B.Cu") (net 2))
 (segment (start 197.54 95.54) (end 203 101) (width 1) (layer "B.Cu") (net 2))
 (segment (start 254.73 90.73) (end 260 90.73) (width 1) (layer "B.Cu") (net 4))
 (segment (start 249.59 80.41) (end 249 81) (width 1) (layer "B.Cu") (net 4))
 (segment (start 249 81) (end 249 85) (width 1) (layer "B.Cu") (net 4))
 (segment (start 249 85) (end 254.73 90.73) (width 1) (layer "B.Cu") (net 4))
 (segment (start 249.59 77.89) (end 249.59 80.41) (width 1) (layer "B.Cu") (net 4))
 (segment (start 260 88.19) (end 252.13 80.32) (width 1) (layer "B.Cu") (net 5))
 (segment (start 252.13 80.32) (end 252.13 77.89) (width 1) (layer "B.Cu") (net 5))
 (segment (start 260.14 81.27) (end 261.37 81.27) (width 1) (layer "B.Cu") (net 35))
 (segment (start 262.64 80) (end 262.64 76.8) (width 1) (layer "B.Cu") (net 35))
 (segment (start 262.64 76.8) (end 260.14 74.3) (width 1) (layer "B.Cu") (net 35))
 (segment (start 261.37 81.27) (end 262.64 80) (width 1) (layer "B.Cu") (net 35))
 (segment (start 260.14 66) (end 254.64 60.5) (width 1) (layer "B.Cu") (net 37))
 (segment (start 254.5 56.5) (end 233 56.5) (width 1) (layer "B.Cu") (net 37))
 (segment (start 233 56.5) (end 231.81 57.69) (width 1) (layer "B.Cu") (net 37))
 (segment (start 260.14 66.68) (end 260.14 66) (width 1) (layer "B.Cu") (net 37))
 (segment (start 231.81 57.69) (end 231.81 59.11) (width 1) (layer "B.Cu") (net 37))
 (segment (start 222 94) (end 211.815 94) (width 1) (layer "B.Cu") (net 8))
 (segment (start 211.8 93.985) (end 216.8 93.985) (width 1) (layer "B.Cu") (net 8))
 (segment (start 211.815 94) (end 211.8 93.985) (width 1) (layer "B.Cu") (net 8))
 (segment (start 206 84) (end 203.87 81.87) (width 1) (layer "B.Cu") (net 16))
 (segment (start 223.27 89.27) (end 218 84) (width 1) (layer "B.Cu") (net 16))
 (segment (start 223.27 94) (end 223.27 89.27) (width 1) (layer "B.Cu") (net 16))
 (segment (start 203.87 81.87) (end 203.87 77.89) (width 1) (layer "B.Cu") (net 16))
 (segment (start 218 84) (end 206 84) (width 1) (layer "B.Cu") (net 16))
 (segment (start 260.14 78.73) (end 257.87 78.73) (width 1) (layer "B.Cu") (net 13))
 (segment (start 195 94) (end 194 95) (width 1) (layer "B.Cu") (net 13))
 (segment (start 255 72) (end 255 61.5) (width 1) (layer "B.Cu") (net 13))
 (segment (start 252.61 59.11) (end 252.13 59.11) (width 1) (layer "B.Cu") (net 13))
 (segment (start 255 61.5) (end 252.61 59.11) (width 1) (layer "B.Cu") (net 13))
 (segment (start 257.87 78.73) (end 255 75.86) (width 1) (layer "B.Cu") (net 13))
 (segment (start 255 75.86) (end 255 71.5) (width 1) (layer "B.Cu") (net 13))
 (segment (start 196.27 77.73) (end 199.5 74.5) (width 1) (layer "B.Cu") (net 14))
 (segment (start 196.27 94) (end 196.27 77.73) (width 1) (layer "B.Cu") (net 14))
 (segment (start 244.51 75.51) (end 244.51 76.89) (width 1) (layer "B.Cu") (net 14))
 (segment (start 243.5 74.5) (end 244.51 75.51) (width 1) (layer "B.Cu") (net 14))
 (segment (start 199.5 74.5) (end 243.5 74.5) (width 1) (layer "B.Cu") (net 14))
 (segment (start 257 80) (end 260.14 80) (width 1) (layer "B.Cu") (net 38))
 (segment (start 236.89 59.11) (end 236.89 62.39) (width 1) (layer "B.Cu") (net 38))
 (segment (start 255 78) (end 257 80) (width 1) (layer "B.Cu") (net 38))
 (segment (start 236.89 62.39) (end 249 74.5) (width 1) (layer "B.Cu") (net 38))
 (segment (start 249 74.5) (end 251.5 74.5) (width 1) (layer "B.Cu") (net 38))
 (segment (start 251.5 74.5) (end 255 78) (width 1) (layer "B.Cu") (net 38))
 (segment (start 214.445 96.525) (end 217 99.08) (width 1) (layer "B.Cu") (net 7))
 (segment (start 211.8 96.525) (end 214.445 96.525) (width 1) (layer "B.Cu") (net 7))
 (segment (start 234.58 53) (end 247 53) (width 1) (layer "B.Cu") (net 15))
 (segment (start 229.27 54.23) (end 229.27 59.11) (width 1) (layer "B.Cu") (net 15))
 (segment (start 249 55) (end 259.735 55) (width 1) (layer "B.Cu") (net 15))
 (segment (start 247 53) (end 249 55) (width 1) (layer "B.Cu") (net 15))
 (segment (start 229.42 58.96) (end 229.27 59.11) (width 1) (layer "B.Cu") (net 15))
 (segment (start 234.58 53) (end 230.5 53) (width 1) (layer "B.Cu") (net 15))
 (segment (start 259.735 55) (end 260 54.735) (width 1) (layer "B.Cu") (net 15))
 (segment (start 230.5 53) (end 229.27 54.23) (width 1) (layer "B.Cu") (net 15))
 (segment (start 229 84) (end 226.73 81.73) (width 1.5) (layer "B.Cu") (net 20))
 (segment (start 226.73 81.73) (end 226.73 77.89) (width 1.5) (layer "B.Cu") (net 20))
 (segment (start 241.5 84) (end 229 84) (width 1.5) (layer "B.Cu") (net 20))
 (segment (start 247.25 89.75) (end 241.5 84) (width 1.5) (layer "B.Cu") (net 20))
 (segment (start 247.25 89.75) (end 247.25 96.25) (width 1.5) (layer "B.Cu") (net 20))
 (segment (start 232 86) (end 235.25 89.25) (width 1.5) (layer "B.Cu") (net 19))
 (segment (start 235.25 89.25) (end 235.25 89.75) (width 1.5) (layer "B.Cu") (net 19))
 (segment (start 235.25 89.75) (end 235.25 96.25) (width 1.5) (layer "B.Cu") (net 19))
 (segment (start 224.19 82.19) (end 228 86) (width 1.5) (layer "B.Cu") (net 19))
 (segment (start 228 86) (end 232 86) (width 1.5) (layer "B.Cu") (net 19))
 (segment (start 224.19 77.89) (end 224.19 82.19) (width 1.5) (layer "B.Cu") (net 19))
 (segment (start 221.65 55.35) (end 221.65 59.11) (width 1) (layer "B.Cu") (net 3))
 (segment (start 232 98) (end 241 98) (width 1) (layer "B.Cu") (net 3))
 (segment (start 208.95 66.05) (end 206 69) (width 1) (layer "B.Cu") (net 3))
 (segment (start 255.27 93.27) (end 260 93.27) (width 1) (layer "B.Cu") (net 3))
 (segment (start 247.05 77.89) (end 247.05 85.05) (width 1) (layer "B.Cu") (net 3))
 (segment (start 227 91) (end 228.25 89.75) (width 1) (layer "B.Cu") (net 3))
 (segment (start 224.54 94) (end 227 91.54) (width 1) (layer "B.Cu") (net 3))
 (segment (start 227 91.54) (end 227 91) (width 1) (layer "B.Cu") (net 3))
 (segment (start 224.42 53) (end 224 53) (width 1) (layer "B.Cu") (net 3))
 (segment (start 208.95 59.11) (end 208.95 66.05) (width 1) (layer "B.Cu") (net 3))
 (segment (start 228.25 89.75) (end 230.75 89.75) (width 1) (layer "B.Cu") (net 3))
 (segment (start 193.12 69) (end 192.2 68.08) (width 1) (layer "B.Cu") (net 3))
 (segment (start 242.75 96.25) (end 242.75 89.75) (width 1) (layer "B.Cu") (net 3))
 (segment (start 224 53) (end 221.65 55.35) (width 1) (layer "B.Cu") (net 3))
 (segment (start 230.75 96.25) (end 230.75 96.75) (width 1) (layer "B.Cu") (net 3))
 (segment (start 230.75 96.75) (end 232 98) (width 1) (layer "B.Cu") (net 3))
 (segment (start 204.1 69) (end 193.12 69) (width 1) (layer "B.Cu") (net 3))
 (segment (start 247.05 85.05) (end 255.27 93.27) (width 1) (layer "B.Cu") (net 3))
 (segment (start 206 69) (end 204.1 69) (width 1) (layer "B.Cu") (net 3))
 (segment (start 241 98) (end 242.75 96.25) (width 1) (layer "B.Cu") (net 3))
 (segment (start 230.75 96.25) (end 230.75 89.75) (width 1) (layer "B.Cu") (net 3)))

